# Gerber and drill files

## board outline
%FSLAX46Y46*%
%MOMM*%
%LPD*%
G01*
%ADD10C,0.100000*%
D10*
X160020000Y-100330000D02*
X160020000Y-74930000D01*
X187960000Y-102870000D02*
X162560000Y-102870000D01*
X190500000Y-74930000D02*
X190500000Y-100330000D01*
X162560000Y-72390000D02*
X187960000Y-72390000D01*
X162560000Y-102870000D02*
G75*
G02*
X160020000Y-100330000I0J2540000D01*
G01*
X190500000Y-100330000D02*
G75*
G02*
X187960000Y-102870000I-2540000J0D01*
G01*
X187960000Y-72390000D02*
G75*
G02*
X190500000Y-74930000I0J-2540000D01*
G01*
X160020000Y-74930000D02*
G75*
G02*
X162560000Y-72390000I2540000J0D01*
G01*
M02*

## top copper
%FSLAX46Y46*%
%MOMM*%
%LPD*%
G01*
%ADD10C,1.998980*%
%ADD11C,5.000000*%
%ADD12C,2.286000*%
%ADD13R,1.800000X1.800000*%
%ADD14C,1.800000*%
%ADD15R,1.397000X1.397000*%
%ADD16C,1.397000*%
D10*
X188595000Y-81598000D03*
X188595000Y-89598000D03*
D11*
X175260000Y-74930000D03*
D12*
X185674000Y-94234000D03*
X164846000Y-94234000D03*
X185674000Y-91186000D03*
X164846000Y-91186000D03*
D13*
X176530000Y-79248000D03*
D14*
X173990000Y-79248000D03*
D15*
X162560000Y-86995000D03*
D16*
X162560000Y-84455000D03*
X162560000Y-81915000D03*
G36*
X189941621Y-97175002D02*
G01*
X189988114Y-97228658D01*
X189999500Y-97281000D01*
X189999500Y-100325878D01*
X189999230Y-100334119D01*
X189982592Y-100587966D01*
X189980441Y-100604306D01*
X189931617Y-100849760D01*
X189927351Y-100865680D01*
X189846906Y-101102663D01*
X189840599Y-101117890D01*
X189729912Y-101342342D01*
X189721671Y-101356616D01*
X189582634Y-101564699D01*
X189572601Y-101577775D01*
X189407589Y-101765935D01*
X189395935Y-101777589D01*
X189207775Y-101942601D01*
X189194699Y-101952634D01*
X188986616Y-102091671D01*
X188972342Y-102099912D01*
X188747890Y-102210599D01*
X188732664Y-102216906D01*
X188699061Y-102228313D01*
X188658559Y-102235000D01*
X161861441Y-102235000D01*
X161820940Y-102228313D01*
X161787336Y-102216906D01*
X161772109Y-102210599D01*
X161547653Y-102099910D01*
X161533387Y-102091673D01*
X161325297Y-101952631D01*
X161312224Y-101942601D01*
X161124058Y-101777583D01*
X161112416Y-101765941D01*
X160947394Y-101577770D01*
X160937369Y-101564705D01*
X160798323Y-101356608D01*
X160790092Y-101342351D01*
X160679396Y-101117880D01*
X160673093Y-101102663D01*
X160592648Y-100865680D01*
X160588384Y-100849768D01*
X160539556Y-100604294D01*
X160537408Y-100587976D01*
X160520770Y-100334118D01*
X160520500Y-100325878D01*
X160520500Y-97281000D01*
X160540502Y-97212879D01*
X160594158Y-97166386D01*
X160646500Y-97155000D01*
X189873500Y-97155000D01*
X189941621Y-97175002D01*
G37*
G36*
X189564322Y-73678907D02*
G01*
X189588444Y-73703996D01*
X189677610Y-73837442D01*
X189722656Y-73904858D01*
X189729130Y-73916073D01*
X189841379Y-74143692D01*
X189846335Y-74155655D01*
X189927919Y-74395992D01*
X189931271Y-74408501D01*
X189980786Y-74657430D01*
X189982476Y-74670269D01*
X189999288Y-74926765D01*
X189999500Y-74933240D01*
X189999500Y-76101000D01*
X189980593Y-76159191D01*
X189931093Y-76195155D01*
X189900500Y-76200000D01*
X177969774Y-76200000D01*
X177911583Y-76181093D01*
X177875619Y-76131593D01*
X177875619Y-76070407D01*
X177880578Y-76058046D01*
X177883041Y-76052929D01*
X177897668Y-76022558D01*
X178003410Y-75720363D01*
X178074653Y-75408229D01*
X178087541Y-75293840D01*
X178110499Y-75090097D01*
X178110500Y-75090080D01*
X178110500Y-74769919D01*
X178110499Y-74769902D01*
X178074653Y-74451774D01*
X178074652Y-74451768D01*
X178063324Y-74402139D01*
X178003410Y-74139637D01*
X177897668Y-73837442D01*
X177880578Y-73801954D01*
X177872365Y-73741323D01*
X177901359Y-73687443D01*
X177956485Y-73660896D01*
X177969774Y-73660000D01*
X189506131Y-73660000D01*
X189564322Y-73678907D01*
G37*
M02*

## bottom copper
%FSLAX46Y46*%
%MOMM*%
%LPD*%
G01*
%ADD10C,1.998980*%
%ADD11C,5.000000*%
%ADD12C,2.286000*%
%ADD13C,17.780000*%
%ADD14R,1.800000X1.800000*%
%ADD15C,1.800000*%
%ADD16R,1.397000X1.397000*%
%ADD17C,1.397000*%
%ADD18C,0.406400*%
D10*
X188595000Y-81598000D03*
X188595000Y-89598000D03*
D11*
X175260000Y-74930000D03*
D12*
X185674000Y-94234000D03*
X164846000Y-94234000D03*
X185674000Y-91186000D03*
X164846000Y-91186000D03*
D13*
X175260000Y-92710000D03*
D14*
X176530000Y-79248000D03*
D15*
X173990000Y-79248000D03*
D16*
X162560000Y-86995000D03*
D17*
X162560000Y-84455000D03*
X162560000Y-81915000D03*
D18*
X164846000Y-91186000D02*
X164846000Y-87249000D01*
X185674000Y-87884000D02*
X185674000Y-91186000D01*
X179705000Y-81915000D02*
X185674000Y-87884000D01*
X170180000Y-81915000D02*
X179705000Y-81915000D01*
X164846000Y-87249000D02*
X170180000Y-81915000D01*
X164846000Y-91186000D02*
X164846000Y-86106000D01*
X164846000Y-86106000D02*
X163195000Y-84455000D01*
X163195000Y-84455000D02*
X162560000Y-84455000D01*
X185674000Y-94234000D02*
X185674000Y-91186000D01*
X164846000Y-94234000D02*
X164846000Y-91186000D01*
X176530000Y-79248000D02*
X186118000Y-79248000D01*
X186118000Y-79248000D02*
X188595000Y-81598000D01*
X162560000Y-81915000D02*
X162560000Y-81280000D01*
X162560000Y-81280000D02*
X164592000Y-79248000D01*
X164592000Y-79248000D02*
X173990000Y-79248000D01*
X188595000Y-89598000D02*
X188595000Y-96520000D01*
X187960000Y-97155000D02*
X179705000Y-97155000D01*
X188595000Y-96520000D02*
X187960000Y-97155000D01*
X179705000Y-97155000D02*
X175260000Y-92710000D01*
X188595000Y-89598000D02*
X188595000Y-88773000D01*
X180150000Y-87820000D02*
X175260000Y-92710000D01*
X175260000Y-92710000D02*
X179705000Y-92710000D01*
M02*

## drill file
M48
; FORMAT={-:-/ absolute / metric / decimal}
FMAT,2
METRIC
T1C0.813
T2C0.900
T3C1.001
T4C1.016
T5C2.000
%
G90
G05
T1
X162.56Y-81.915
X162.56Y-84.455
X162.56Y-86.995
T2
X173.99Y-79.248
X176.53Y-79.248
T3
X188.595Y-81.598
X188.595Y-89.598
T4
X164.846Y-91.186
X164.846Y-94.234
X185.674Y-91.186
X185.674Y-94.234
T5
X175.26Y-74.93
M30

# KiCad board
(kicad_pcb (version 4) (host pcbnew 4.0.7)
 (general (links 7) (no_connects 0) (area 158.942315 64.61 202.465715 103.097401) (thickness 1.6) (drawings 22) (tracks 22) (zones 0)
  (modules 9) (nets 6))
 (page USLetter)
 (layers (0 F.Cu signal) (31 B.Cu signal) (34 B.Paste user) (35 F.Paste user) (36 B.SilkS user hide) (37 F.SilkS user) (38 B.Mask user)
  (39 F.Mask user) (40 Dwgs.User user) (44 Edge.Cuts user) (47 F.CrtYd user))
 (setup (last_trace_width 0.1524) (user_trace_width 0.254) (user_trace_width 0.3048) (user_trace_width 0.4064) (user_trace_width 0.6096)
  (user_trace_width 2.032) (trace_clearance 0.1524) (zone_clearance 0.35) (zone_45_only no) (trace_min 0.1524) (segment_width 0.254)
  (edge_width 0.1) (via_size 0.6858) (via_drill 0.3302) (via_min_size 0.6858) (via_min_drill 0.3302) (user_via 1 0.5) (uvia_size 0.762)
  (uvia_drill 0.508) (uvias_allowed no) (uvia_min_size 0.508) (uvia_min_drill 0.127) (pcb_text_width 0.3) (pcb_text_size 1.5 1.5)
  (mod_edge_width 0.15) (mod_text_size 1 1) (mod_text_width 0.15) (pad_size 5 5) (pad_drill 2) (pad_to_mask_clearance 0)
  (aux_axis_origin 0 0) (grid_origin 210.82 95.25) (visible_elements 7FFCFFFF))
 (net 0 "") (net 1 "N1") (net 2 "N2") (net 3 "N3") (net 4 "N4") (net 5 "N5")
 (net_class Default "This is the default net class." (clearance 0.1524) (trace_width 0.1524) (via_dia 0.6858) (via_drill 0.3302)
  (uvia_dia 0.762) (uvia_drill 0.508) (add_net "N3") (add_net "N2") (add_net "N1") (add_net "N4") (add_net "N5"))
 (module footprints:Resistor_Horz (layer F.Cu) (at 188.595 85.598 270)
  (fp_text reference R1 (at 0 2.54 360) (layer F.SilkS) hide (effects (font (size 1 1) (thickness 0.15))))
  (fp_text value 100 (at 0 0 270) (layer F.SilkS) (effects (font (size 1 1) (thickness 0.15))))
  (pad 1 thru_hole circle (at -4 0 270) (size 1.99898 1.99898) (drill 1.00076) (layers *.Cu *.SilkS *.Mask) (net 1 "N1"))
  (pad 2 thru_hole circle (at 4 0 270) (size 1.99898 1.99898) (drill 1.00076) (layers *.Cu *.SilkS *.Mask) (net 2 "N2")))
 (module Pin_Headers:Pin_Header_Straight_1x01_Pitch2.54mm (layer F.Cu) (at 175.26 74.93)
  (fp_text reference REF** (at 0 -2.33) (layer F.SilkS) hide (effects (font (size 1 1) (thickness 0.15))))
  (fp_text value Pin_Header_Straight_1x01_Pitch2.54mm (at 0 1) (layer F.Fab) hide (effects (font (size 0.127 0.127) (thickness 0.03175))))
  (pad 1 thru_hole circle (at 0 0) (size 5 5) (drill 2) (layers *.Cu B.Mask)))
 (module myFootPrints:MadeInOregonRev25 (layer F.Cu) (at 167.64 76.454)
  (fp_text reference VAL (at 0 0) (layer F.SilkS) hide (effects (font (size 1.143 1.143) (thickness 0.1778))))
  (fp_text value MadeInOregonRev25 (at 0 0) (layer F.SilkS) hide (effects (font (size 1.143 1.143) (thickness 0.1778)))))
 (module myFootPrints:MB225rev (layer F.Cu) (at 184.15 76.2)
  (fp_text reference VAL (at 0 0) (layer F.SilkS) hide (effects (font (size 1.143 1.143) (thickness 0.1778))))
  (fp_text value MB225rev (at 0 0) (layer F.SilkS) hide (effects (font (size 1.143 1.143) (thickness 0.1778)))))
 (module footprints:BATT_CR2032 (layer B.Cu) (at 175.26 92.71 180)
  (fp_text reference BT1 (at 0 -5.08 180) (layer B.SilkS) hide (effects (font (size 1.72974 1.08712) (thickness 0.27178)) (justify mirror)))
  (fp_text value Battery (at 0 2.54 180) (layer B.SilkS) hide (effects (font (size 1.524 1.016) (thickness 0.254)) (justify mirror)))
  (pad 1 thru_hole circle (at -10.414 -1.524 180) (size 2.286 2.286) (drill 1.016) (layers *.Cu *.Mask B.SilkS) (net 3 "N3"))
  (pad 1 thru_hole circle (at 10.414 -1.524 180) (size 2.286 2.286) (drill 1.016) (layers *.Cu *.Mask B.SilkS) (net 3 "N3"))
  (pad 1 thru_hole circle (at -10.414 1.524 180) (size 2.286 2.286) (drill 1.016) (layers *.Cu *.Mask B.SilkS) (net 3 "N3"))
  (pad 1 thru_hole circle (at 10.414 1.524 180) (size 2.286 2.286) (drill 1.016) (layers *.Cu *.Mask B.SilkS) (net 3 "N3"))
  (pad 2 smd circle (at 0 0 180) (size 17.78 17.78) (layers B.Cu B.Paste B.Mask) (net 2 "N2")))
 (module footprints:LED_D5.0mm (layer F.Cu) (at 176.53 79.248 180)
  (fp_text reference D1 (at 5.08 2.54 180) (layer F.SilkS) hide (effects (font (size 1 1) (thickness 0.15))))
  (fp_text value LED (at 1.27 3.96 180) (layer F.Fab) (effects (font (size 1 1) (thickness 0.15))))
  (pad 1 thru_hole rect (at 0 0 180) (size 1.8 1.8) (drill 0.9) (layers *.Cu *.Mask) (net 1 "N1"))
  (pad 2 thru_hole circle (at 2.54 0 180) (size 1.8 1.8) (drill 0.9) (layers *.Cu *.Mask) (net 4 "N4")))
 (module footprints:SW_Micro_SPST (layer F.Cu) (at 162.56 84.455 90)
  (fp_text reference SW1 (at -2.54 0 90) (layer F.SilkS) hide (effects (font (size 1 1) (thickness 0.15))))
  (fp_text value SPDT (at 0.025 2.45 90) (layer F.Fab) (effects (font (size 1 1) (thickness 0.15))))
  (pad 1 thru_hole rect (at -2.54 0 90) (size 1.397 1.397) (drill 0.8128) (layers *.Cu *.Mask F.SilkS) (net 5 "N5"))
  (pad 2 thru_hole circle (at 0 0 90) (size 1.397 1.397) (drill 0.8128) (layers *.Cu *.Mask F.SilkS) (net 3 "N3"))
  (pad 3 thru_hole circle (at 2.54 0 90) (size 1.397 1.397) (drill 0.8128) (layers *.Cu *.Mask F.SilkS) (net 4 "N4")))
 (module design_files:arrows (layer F.Cu) (at 179.07 77.47)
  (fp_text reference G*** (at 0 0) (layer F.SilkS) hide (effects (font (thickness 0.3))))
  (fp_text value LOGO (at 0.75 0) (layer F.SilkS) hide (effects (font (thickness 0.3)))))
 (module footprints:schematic (layer F.Cu) (at 175.26 87.503)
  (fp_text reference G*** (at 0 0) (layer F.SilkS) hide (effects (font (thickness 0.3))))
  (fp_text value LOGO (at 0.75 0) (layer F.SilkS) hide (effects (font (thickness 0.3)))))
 (gr_line (start 160.02 100.33) (end 160.02 74.93) (angle 90) (layer Edge.Cuts) (width 0.1))
 (gr_line (start 187.96 102.87) (end 162.56 102.87) (angle 90) (layer Edge.Cuts) (width 0.1))
 (gr_line (start 190.5 74.93) (end 190.5 100.33) (angle 90) (layer Edge.Cuts) (width 0.1))
 (gr_line (start 162.56 72.39) (end 187.96 72.39) (angle 90) (layer Edge.Cuts) (width 0.1))
 (gr_arc (start 162.56 100.33) (end 162.56 102.87) (angle 90) (layer Edge.Cuts) (width 0.1))
 (gr_arc (start 187.96 100.33) (end 190.5 100.33) (angle 90) (layer Edge.Cuts) (width 0.1))
 (gr_arc (start 187.96 74.93) (end 187.96 72.39) (angle 90) (layer Edge.Cuts) (width 0.1))
 (gr_arc (start 162.56 74.93) (end 160.02 74.93) (angle 90) (layer Edge.Cuts) (width 0.1))
 (segment (start 164.846 91.186) (end 164.846 87.249) (width 0.4064) (layer B.Cu) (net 3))
 (segment (start 185.674 87.884) (end 185.674 91.186) (width 0.4064) (layer B.Cu) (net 3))
 (segment (start 179.705 81.915) (end 185.674 87.884) (width 0.4064) (layer B.Cu) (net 3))
 (segment (start 170.18 81.915) (end 179.705 81.915) (width 0.4064) (layer B.Cu) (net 3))
 (segment (start 164.846 87.249) (end 170.18 81.915) (width 0.4064) (layer B.Cu) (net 3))
 (segment (start 164.846 91.186) (end 164.846 86.106) (width 0.4064) (layer B.Cu) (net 3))
 (segment (start 164.846 86.106) (end 163.195 84.455) (width 0.4064) (layer B.Cu) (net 3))
 (segment (start 163.195 84.455) (end 162.56 84.455) (width 0.4064) (layer B.Cu) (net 3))
 (segment (start 185.674 94.234) (end 185.674 91.186) (width 0.4064) (layer B.Cu) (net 3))
 (segment (start 164.846 94.234) (end 164.846 91.186) (width 0.4064) (layer B.Cu) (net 3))
 (segment (start 176.53 79.248) (end 186.118 79.248) (width 0.4064) (layer B.Cu) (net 1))
 (segment (start 186.118 79.248) (end 188.595 81.598) (width 0.4064) (layer B.Cu) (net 1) (status 20))
 (segment (start 162.56 81.915) (end 162.56 81.28) (width 0.4064) (layer B.Cu) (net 4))
 (segment (start 162.56 81.28) (end 164.592 79.248) (width 0.4064) (layer B.Cu) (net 4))
 (segment (start 164.592 79.248) (end 173.99 79.248) (width 0.4064) (layer B.Cu) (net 4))
 (segment (start 188.595 89.598) (end 188.595 96.52) (width 0.4064) (layer B.Cu) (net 2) (status 10))
 (segment (start 187.96 97.155) (end 179.705 97.155) (width 0.4064) (layer B.Cu) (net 2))
 (segment (start 188.595 96.52) (end 187.96 97.155) (width 0.4064) (layer B.Cu) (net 2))
 (segment (start 179.705 97.155) (end 175.26 92.71) (width 0.4064) (layer B.Cu) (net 2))
 (segment (start 188.595 89.598) (end 188.595 88.773) (width 0.4064) (layer B.Cu) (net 2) (status 30))
 (segment (start 180.15 87.82) (end 175.26 92.71) (width 0.4064) (layer B.Cu) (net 2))
 (segment (start 175.26 92.71) (end 179.705 92.71) (width 0.4064) (layer B.Cu) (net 2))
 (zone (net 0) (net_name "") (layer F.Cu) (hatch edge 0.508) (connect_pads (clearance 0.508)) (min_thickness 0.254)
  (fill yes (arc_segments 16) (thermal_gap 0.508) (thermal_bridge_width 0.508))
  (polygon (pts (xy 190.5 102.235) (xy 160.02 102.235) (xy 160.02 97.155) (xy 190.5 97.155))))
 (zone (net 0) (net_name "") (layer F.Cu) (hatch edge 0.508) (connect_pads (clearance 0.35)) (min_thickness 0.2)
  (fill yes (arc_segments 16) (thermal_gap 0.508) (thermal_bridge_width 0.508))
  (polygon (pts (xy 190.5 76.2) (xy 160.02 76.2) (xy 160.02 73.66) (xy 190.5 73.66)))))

